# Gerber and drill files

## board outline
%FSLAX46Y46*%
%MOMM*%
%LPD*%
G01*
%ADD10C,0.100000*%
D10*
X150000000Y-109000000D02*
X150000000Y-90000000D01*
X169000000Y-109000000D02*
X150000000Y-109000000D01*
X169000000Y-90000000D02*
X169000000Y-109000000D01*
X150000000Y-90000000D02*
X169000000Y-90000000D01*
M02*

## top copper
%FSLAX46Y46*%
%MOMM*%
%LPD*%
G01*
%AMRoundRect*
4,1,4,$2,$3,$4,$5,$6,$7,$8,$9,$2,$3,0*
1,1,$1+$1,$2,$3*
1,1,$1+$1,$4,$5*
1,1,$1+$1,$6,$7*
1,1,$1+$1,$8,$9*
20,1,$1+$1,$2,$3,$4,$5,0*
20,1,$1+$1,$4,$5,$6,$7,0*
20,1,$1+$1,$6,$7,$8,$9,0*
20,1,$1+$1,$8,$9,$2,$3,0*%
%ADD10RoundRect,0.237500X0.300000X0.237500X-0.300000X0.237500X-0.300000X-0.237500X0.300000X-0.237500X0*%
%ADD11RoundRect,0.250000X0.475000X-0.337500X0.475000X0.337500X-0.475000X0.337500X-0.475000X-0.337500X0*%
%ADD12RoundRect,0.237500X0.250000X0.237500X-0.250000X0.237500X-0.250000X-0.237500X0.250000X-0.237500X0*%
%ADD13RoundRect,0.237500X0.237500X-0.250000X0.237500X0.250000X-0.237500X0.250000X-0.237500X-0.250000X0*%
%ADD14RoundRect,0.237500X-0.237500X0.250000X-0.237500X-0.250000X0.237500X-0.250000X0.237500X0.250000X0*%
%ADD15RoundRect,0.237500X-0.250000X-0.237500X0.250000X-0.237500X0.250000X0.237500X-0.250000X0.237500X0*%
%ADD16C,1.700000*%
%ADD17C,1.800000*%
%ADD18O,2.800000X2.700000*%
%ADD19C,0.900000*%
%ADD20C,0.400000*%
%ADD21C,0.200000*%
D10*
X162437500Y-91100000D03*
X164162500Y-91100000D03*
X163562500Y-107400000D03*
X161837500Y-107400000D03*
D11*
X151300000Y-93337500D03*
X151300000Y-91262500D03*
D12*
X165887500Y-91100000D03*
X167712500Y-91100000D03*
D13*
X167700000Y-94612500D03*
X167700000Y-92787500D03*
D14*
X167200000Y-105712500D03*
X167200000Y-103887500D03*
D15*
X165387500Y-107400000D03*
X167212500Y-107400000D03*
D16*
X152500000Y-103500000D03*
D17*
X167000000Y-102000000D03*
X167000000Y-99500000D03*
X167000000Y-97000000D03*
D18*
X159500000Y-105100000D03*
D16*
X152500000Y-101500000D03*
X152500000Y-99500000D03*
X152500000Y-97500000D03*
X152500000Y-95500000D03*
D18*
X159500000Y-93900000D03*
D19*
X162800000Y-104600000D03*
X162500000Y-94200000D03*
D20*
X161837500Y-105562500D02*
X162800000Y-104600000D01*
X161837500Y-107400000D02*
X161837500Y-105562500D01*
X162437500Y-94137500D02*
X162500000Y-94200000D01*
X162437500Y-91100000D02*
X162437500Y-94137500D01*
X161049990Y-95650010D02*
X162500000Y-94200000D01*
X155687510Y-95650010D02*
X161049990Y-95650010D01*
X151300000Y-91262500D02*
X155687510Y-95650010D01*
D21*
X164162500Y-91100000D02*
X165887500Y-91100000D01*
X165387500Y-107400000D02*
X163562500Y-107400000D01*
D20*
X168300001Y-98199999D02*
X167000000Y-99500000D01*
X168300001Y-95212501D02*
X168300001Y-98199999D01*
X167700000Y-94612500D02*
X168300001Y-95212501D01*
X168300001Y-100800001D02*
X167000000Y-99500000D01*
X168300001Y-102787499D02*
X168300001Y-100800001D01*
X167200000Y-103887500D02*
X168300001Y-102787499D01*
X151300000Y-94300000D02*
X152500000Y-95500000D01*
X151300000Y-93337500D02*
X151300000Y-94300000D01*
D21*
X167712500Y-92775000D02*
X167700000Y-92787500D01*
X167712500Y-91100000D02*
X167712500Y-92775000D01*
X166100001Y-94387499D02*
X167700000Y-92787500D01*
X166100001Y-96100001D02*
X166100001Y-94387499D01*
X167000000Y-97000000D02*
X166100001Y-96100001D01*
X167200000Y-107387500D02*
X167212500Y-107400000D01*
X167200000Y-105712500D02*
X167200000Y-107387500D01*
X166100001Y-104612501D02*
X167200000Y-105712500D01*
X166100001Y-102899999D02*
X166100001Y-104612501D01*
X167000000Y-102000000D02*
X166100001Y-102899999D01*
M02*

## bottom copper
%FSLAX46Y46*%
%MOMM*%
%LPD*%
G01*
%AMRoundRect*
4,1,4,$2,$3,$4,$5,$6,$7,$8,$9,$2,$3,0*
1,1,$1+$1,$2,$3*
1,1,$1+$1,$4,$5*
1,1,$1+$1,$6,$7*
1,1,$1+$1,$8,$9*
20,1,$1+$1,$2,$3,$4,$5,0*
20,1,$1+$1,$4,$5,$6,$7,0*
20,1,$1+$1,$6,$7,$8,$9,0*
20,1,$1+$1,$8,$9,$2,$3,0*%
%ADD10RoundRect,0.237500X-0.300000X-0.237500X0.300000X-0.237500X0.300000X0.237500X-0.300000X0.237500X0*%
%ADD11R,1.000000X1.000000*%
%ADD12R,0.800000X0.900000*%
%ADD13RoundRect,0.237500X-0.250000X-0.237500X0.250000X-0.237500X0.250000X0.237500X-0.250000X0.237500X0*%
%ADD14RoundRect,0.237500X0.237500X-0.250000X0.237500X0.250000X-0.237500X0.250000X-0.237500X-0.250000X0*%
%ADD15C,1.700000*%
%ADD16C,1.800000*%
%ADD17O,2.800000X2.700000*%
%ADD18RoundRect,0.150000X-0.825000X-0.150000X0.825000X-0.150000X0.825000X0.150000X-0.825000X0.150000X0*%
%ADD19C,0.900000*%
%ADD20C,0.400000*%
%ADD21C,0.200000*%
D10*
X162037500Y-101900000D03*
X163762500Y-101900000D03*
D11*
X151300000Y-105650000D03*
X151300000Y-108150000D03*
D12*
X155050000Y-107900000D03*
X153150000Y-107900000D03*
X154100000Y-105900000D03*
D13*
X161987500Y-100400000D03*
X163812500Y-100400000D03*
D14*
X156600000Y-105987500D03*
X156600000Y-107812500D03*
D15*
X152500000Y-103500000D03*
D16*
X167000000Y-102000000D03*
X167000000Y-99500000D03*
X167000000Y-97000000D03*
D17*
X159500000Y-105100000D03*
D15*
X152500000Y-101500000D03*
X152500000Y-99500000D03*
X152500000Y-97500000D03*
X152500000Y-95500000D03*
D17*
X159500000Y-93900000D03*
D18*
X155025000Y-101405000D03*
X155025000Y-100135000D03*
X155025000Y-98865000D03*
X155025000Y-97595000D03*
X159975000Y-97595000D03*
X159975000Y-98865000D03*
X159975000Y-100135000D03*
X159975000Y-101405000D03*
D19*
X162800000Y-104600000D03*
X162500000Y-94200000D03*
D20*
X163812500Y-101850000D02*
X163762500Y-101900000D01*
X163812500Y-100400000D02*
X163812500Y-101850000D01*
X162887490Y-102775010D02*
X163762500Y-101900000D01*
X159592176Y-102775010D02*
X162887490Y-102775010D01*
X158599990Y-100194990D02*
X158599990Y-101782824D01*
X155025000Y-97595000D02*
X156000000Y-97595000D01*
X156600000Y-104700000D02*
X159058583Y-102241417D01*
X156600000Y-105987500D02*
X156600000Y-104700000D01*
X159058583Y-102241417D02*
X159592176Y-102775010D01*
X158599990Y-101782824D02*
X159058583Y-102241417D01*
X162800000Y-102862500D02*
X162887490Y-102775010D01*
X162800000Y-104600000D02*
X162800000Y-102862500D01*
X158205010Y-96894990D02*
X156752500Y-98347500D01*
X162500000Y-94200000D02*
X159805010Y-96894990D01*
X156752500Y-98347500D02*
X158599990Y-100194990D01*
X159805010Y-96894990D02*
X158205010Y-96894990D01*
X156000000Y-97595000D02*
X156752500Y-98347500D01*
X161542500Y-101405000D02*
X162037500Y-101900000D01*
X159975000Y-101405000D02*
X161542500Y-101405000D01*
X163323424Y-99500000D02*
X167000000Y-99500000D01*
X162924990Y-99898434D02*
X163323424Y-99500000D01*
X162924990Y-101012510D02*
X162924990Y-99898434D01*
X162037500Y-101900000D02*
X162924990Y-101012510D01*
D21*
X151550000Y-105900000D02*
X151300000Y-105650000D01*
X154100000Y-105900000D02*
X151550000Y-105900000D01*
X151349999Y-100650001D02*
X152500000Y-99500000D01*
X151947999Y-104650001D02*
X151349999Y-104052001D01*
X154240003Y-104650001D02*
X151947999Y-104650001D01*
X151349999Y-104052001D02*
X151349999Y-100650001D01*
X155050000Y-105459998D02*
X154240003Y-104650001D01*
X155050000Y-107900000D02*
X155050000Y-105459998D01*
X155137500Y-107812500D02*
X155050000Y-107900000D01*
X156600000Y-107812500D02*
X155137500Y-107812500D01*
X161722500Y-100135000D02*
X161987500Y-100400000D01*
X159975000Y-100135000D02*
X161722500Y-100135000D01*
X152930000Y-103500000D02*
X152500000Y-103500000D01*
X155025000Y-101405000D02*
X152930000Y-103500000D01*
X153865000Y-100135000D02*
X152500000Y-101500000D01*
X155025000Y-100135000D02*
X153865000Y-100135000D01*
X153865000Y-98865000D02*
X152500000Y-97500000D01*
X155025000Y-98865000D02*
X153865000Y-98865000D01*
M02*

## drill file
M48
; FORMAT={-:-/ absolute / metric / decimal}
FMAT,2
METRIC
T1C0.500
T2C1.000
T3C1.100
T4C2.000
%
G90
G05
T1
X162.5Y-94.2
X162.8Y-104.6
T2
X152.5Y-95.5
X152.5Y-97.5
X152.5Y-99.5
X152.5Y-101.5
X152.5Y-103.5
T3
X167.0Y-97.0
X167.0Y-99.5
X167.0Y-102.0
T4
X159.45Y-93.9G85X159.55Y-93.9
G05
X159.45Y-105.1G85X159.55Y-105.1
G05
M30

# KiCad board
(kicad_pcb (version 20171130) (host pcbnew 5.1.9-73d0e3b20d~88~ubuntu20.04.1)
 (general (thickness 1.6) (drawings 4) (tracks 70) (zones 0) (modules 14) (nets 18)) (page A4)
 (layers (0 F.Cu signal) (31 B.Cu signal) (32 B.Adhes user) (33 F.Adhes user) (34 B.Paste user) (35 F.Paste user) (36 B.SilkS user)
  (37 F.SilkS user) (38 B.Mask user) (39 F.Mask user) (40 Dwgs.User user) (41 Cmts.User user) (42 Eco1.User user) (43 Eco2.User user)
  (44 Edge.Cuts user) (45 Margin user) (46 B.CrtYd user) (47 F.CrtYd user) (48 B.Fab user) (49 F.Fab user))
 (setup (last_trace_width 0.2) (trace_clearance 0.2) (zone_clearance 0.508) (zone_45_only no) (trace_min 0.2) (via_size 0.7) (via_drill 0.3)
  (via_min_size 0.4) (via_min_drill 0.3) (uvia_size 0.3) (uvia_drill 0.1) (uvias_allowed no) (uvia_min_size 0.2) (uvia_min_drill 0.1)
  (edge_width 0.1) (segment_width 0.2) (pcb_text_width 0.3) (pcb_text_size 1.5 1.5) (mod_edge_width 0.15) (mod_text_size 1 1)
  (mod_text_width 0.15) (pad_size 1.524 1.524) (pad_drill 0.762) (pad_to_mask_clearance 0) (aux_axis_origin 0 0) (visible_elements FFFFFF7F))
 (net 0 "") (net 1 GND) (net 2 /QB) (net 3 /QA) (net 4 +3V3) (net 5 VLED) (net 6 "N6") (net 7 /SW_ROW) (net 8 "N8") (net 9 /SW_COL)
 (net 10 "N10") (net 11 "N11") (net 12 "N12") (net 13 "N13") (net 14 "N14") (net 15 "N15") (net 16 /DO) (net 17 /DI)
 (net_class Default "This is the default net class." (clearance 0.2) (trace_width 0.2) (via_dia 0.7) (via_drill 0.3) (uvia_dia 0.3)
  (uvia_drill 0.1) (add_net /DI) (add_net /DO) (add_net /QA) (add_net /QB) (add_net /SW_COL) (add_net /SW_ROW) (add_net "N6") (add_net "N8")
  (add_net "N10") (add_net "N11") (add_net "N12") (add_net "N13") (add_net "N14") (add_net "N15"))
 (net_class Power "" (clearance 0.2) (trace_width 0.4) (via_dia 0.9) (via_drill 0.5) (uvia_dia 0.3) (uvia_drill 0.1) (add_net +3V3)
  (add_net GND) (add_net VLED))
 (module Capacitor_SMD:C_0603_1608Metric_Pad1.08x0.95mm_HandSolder (layer F.Cu) (at 163.3 91.1 180)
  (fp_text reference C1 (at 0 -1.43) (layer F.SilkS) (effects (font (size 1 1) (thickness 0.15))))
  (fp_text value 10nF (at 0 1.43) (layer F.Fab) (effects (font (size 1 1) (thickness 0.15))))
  (pad 2 smd roundrect (at 0.8625 0 180) (size 1.075 0.95) (layers F.Cu F.Paste F.Mask) (roundrect_rratio 0.25) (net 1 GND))
  (pad 1 smd roundrect (at -0.8625 0 180) (size 1.075 0.95) (layers F.Cu F.Paste F.Mask) (roundrect_rratio 0.25) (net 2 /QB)))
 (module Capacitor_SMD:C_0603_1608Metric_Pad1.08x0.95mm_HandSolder (layer F.Cu) (at 162.7 107.4 180)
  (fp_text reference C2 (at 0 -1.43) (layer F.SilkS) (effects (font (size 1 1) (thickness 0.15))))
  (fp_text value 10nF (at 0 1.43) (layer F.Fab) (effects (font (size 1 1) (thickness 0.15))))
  (pad 1 smd roundrect (at -0.8625 0 180) (size 1.075 0.95) (layers F.Cu F.Paste F.Mask) (roundrect_rratio 0.25) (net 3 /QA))
  (pad 2 smd roundrect (at 0.8625 0 180) (size 1.075 0.95) (layers F.Cu F.Paste F.Mask) (roundrect_rratio 0.25) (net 1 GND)))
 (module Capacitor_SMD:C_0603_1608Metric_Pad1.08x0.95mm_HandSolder (layer B.Cu) (at 162.9 101.9)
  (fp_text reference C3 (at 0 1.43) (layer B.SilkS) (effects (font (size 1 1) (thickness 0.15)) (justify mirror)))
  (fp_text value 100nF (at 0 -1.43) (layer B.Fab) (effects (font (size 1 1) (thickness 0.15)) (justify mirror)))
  (pad 1 smd roundrect (at -0.8625 0) (size 1.075 0.95) (layers B.Cu B.Paste B.Mask) (roundrect_rratio 0.25) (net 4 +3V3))
  (pad 2 smd roundrect (at 0.8625 0) (size 1.075 0.95) (layers B.Cu B.Paste B.Mask) (roundrect_rratio 0.25) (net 1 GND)))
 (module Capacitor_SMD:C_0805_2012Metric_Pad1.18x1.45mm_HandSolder (layer F.Cu) (at 151.3 92.3 90)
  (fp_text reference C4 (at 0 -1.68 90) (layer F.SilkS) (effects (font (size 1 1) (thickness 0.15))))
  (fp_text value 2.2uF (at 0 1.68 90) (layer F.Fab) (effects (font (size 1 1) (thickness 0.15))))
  (pad 1 smd roundrect (at -1.0375 0 90) (size 1.175 1.45) (layers F.Cu F.Paste F.Mask) (roundrect_rratio 0.212766) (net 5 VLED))
  (pad 2 smd roundrect (at 1.0375 0 90) (size 1.175 1.45) (layers F.Cu F.Paste F.Mask) (roundrect_rratio 0.212766) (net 1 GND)))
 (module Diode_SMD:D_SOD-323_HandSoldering (layer B.Cu) (at 151.3 106.9 270)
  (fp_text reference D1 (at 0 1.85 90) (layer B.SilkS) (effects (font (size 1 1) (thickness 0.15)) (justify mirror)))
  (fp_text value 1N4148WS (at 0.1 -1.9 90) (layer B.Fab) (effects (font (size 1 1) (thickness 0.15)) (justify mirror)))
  (pad 1 smd rect (at -1.25 0 270) (size 1 1) (layers B.Cu B.Paste B.Mask) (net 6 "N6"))
  (pad 2 smd rect (at 1.25 0 270) (size 1 1) (layers B.Cu B.Paste B.Mask) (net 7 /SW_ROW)))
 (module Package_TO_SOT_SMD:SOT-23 (layer B.Cu) (at 154.1 106.9 90)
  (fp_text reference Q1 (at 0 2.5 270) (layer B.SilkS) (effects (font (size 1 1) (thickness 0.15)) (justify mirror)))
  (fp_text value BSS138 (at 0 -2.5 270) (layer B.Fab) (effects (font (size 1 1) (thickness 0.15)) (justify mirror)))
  (pad 1 smd rect (at -1 0.95 90) (size 0.9 0.8) (layers B.Cu B.Paste B.Mask) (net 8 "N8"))
  (pad 2 smd rect (at -1 -0.95 90) (size 0.9 0.8) (layers B.Cu B.Paste B.Mask) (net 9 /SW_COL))
  (pad 3 smd rect (at 1 0 90) (size 0.9 0.8) (layers B.Cu B.Paste B.Mask) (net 6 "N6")))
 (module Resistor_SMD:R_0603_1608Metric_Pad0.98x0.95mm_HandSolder (layer F.Cu) (at 166.8 91.1 180)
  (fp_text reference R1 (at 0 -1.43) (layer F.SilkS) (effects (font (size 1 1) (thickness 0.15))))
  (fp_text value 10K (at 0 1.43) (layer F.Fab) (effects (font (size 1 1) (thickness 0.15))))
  (pad 2 smd roundrect (at 0.9125 0 180) (size 0.975 0.95) (layers F.Cu F.Paste F.Mask) (roundrect_rratio 0.25) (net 2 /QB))
  (pad 1 smd roundrect (at -0.9125 0 180) (size 0.975 0.95) (layers F.Cu F.Paste F.Mask) (roundrect_rratio 0.25) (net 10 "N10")))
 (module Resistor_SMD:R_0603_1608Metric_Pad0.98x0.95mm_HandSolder (layer F.Cu) (at 167.7 93.7 90)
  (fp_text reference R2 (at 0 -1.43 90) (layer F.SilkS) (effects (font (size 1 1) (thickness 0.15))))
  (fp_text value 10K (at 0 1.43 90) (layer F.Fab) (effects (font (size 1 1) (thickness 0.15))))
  (pad 1 smd roundrect (at -0.9125 0 90) (size 0.975 0.95) (layers F.Cu F.Paste F.Mask) (roundrect_rratio 0.25) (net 4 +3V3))
  (pad 2 smd roundrect (at 0.9125 0 90) (size 0.975 0.95) (layers F.Cu F.Paste F.Mask) (roundrect_rratio 0.25) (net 10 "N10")))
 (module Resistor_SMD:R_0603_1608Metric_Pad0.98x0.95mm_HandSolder (layer B.Cu) (at 162.9 100.4)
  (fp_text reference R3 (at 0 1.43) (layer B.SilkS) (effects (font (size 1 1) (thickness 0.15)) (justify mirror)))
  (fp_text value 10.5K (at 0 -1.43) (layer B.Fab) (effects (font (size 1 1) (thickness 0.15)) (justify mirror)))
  (pad 1 smd roundrect (at -0.9125 0) (size 0.975 0.95) (layers B.Cu B.Paste B.Mask) (roundrect_rratio 0.25) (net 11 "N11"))
  (pad 2 smd roundrect (at 0.9125 0) (size 0.975 0.95) (layers B.Cu B.Paste B.Mask) (roundrect_rratio 0.25) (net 1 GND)))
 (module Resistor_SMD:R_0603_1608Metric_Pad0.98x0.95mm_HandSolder (layer F.Cu) (at 167.2 104.8 270)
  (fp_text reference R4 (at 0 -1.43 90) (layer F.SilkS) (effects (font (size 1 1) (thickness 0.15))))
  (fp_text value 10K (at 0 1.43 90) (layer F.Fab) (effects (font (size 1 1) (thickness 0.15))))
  (pad 2 smd roundrect (at 0.9125 0 270) (size 0.975 0.95) (layers F.Cu F.Paste F.Mask) (roundrect_rratio 0.25) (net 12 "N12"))
  (pad 1 smd roundrect (at -0.9125 0 270) (size 0.975 0.95) (layers F.Cu F.Paste F.Mask) (roundrect_rratio 0.25) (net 4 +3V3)))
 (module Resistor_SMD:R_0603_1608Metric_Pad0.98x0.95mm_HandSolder (layer F.Cu) (at 166.3 107.4)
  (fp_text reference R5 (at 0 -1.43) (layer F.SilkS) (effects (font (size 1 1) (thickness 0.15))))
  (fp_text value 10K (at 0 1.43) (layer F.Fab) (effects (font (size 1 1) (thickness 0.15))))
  (pad 1 smd roundrect (at -0.9125 0) (size 0.975 0.95) (layers F.Cu F.Paste F.Mask) (roundrect_rratio 0.25) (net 3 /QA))
  (pad 2 smd roundrect (at 0.9125 0) (size 0.975 0.95) (layers F.Cu F.Paste F.Mask) (roundrect_rratio 0.25) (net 12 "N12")))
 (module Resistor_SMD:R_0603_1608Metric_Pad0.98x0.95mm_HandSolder (layer B.Cu) (at 156.6 106.9 90)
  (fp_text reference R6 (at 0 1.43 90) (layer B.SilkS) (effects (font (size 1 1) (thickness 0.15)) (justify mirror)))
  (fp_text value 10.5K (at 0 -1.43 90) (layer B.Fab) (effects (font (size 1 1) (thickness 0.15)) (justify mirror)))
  (pad 2 smd roundrect (at 0.9125 0 90) (size 0.975 0.95) (layers B.Cu B.Paste B.Mask) (roundrect_rratio 0.25) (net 1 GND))
  (pad 1 smd roundrect (at -0.9125 0 90) (size 0.975 0.95) (layers B.Cu B.Paste B.Mask) (roundrect_rratio 0.25) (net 8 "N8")))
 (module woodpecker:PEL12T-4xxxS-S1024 (layer F.Cu) (at 159.5 99.5 90)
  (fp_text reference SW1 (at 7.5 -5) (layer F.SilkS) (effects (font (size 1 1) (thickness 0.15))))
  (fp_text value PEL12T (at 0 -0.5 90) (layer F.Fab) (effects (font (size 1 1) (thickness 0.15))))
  (pad 1 thru_hole circle (at -4 -7 90) (size 1.7 1.7) (drill 1) (layers *.Cu *.Mask) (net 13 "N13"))
  (pad A thru_hole circle (at -2.5 7.5 90) (size 1.8 1.8) (drill 1.1) (layers *.Cu *.Mask) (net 12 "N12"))
  (pad C thru_hole circle (at 0 7.5 90) (size 1.8 1.8) (drill 1.1) (layers *.Cu *.Mask) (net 4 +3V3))
  (pad B thru_hole circle (at 2.5 7.5 90) (size 1.8 1.8) (drill 1.1) (layers *.Cu *.Mask) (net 10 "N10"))
  (pad "" np_thru_hole oval (at -5.6 0 90) (size 2.7 2.8) (drill oval 2 2.1) (layers *.Cu *.Mask))
  (pad 2 thru_hole circle (at -2 -7 90) (size 1.7 1.7) (drill 1) (layers *.Cu *.Mask) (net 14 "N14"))
  (pad 3 thru_hole circle (at 0 -7 90) (size 1.7 1.7) (drill 1) (layers *.Cu *.Mask) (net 8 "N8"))
  (pad 4 thru_hole circle (at 2 -7 90) (size 1.7 1.7) (drill 1) (layers *.Cu *.Mask) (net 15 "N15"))
  (pad 5 thru_hole circle (at 4 -7 90) (size 1.7 1.7) (drill 1) (layers *.Cu *.Mask) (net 5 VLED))
  (pad "" np_thru_hole oval (at 5.6 0 90) (size 2.7 2.8) (drill oval 2 2.1) (layers *.Cu *.Mask)))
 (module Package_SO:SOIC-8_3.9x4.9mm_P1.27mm (layer B.Cu) (at 157.5 99.5)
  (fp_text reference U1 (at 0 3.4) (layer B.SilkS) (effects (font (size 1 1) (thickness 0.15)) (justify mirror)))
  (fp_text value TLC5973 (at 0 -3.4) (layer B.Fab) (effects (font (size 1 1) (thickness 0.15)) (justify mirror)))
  (pad 1 smd roundrect (at -2.475 1.905) (size 1.95 0.6) (layers B.Cu B.Paste B.Mask) (roundrect_rratio 0.25) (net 13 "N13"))
  (pad 2 smd roundrect (at -2.475 0.635) (size 1.95 0.6) (layers B.Cu B.Paste B.Mask) (roundrect_rratio 0.25) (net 14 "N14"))
  (pad 3 smd roundrect (at -2.475 -0.635) (size 1.95 0.6) (layers B.Cu B.Paste B.Mask) (roundrect_rratio 0.25) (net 15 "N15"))
  (pad 4 smd roundrect (at -2.475 -1.905) (size 1.95 0.6) (layers B.Cu B.Paste B.Mask) (roundrect_rratio 0.25) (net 1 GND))
  (pad 5 smd roundrect (at 2.475 -1.905) (size 1.95 0.6) (layers B.Cu B.Paste B.Mask) (roundrect_rratio 0.25) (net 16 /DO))
  (pad 6 smd roundrect (at 2.475 -0.635) (size 1.95 0.6) (layers B.Cu B.Paste B.Mask) (roundrect_rratio 0.25) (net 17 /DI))
  (pad 7 smd roundrect (at 2.475 0.635) (size 1.95 0.6) (layers B.Cu B.Paste B.Mask) (roundrect_rratio 0.25) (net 11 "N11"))
  (pad 8 smd roundrect (at 2.475 1.905) (size 1.95 0.6) (layers B.Cu B.Paste B.Mask) (roundrect_rratio 0.25) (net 4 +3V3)))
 (gr_line (start 150 109) (end 150 90) (layer Edge.Cuts) (width 0.1))
 (gr_line (start 169 109) (end 150 109) (layer Edge.Cuts) (width 0.1))
 (gr_line (start 169 90) (end 169 109) (layer Edge.Cuts) (width 0.1))
 (gr_line (start 150 90) (end 169 90) (layer Edge.Cuts) (width 0.1))
 (segment (start 163.8125 101.85) (end 163.7625 101.9) (width 0.4) (layer B.Cu) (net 1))
 (segment (start 163.8125 100.4) (end 163.8125 101.85) (width 0.4) (layer B.Cu) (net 1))
 (segment (start 162.88749 102.77501) (end 163.7625 101.9) (width 0.4) (layer B.Cu) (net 1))
 (segment (start 159.592176 102.77501) (end 162.88749 102.77501) (width 0.4) (layer B.Cu) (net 1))
 (segment (start 158.59999 100.19499) (end 158.59999 101.782824) (width 0.4) (layer B.Cu) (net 1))
 (segment (start 155.025 97.595) (end 156 97.595) (width 0.4) (layer B.Cu) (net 1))
 (segment (start 156.6 104.7) (end 159.058583 102.241417) (width 0.4) (layer B.Cu) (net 1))
 (segment (start 156.6 105.9875) (end 156.6 104.7) (width 0.4) (layer B.Cu) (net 1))
 (segment (start 159.058583 102.241417) (end 159.592176 102.77501) (width 0.4) (layer B.Cu) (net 1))
 (segment (start 158.59999 101.782824) (end 159.058583 102.241417) (width 0.4) (layer B.Cu) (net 1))
 (via (at 162.8 104.6) (size 0.9) (drill 0.5) (layers F.Cu B.Cu) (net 1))
 (segment (start 161.8375 105.5625) (end 162.8 104.6) (width 0.4) (layer F.Cu) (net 1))
 (segment (start 161.8375 107.4) (end 161.8375 105.5625) (width 0.4) (layer F.Cu) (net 1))
 (segment (start 162.8 102.8625) (end 162.88749 102.77501) (width 0.4) (layer B.Cu) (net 1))
 (segment (start 162.8 104.6) (end 162.8 102.8625) (width 0.4) (layer B.Cu) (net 1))
 (via (at 162.5 94.2) (size 0.9) (drill 0.5) (layers F.Cu B.Cu) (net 1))
 (segment (start 162.4375 94.1375) (end 162.5 94.2) (width 0.4) (layer F.Cu) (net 1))
 (segment (start 162.4375 91.1) (end 162.4375 94.1375) (width 0.4) (layer F.Cu) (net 1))
 (segment (start 158.20501 96.89499) (end 156.7525 98.3475) (width 0.4) (layer B.Cu) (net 1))
 (segment (start 162.5 94.2) (end 159.80501 96.89499) (width 0.4) (layer B.Cu) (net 1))
 (segment (start 156.7525 98.3475) (end 158.59999 100.19499) (width 0.4) (layer B.Cu) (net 1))
 (segment (start 159.80501 96.89499) (end 158.20501 96.89499) (width 0.4) (layer B.Cu) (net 1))
 (segment (start 156 97.595) (end 156.7525 98.3475) (width 0.4) (layer B.Cu) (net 1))
 (segment (start 161.04999 95.65001) (end 162.5 94.2) (width 0.4) (layer F.Cu) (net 1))
 (segment (start 155.68751 95.65001) (end 161.04999 95.65001) (width 0.4) (layer F.Cu) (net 1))
 (segment (start 151.3 91.2625) (end 155.68751 95.65001) (width 0.4) (layer F.Cu) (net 1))
 (segment (start 164.1625 91.1) (end 165.8875 91.1) (width 0.2) (layer F.Cu) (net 2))
 (segment (start 165.3875 107.4) (end 163.5625 107.4) (width 0.2) (layer F.Cu) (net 3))
 (segment (start 161.5425 101.405) (end 162.0375 101.9) (width 0.4) (layer B.Cu) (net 4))
 (segment (start 159.975 101.405) (end 161.5425 101.405) (width 0.4) (layer B.Cu) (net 4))
 (segment (start 163.323424 99.5) (end 167 99.5) (width 0.4) (layer B.Cu) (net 4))
 (segment (start 162.92499 99.898434) (end 163.323424 99.5) (width 0.4) (layer B.Cu) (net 4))
 (segment (start 162.92499 101.01251) (end 162.92499 99.898434) (width 0.4) (layer B.Cu) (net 4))
 (segment (start 162.0375 101.9) (end 162.92499 101.01251) (width 0.4) (layer B.Cu) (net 4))
 (segment (start 168.300001 98.199999) (end 167 99.5) (width 0.4) (layer F.Cu) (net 4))
 (segment (start 168.300001 95.212501) (end 168.300001 98.199999) (width 0.4) (layer F.Cu) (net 4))
 (segment (start 167.7 94.6125) (end 168.300001 95.212501) (width 0.4) (layer F.Cu) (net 4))
 (segment (start 168.300001 100.800001) (end 167 99.5) (width 0.4) (layer F.Cu) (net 4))
 (segment (start 168.300001 102.787499) (end 168.300001 100.800001) (width 0.4) (layer F.Cu) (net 4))
 (segment (start 167.2 103.8875) (end 168.300001 102.787499) (width 0.4) (layer F.Cu) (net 4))
 (segment (start 151.3 94.3) (end 152.5 95.5) (width 0.4) (layer F.Cu) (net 5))
 (segment (start 151.3 93.3375) (end 151.3 94.3) (width 0.4) (layer F.Cu) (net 5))
 (segment (start 151.55 105.9) (end 151.3 105.65) (width 0.2) (layer B.Cu) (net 6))
 (segment (start 154.1 105.9) (end 151.55 105.9) (width 0.2) (layer B.Cu) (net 6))
 (segment (start 151.349999 100.650001) (end 152.5 99.5) (width 0.2) (layer B.Cu) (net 8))
 (segment (start 151.947999 104.650001) (end 151.349999 104.052001) (width 0.2) (layer B.Cu) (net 8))
 (segment (start 154.240003 104.650001) (end 151.947999 104.650001) (width 0.2) (layer B.Cu) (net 8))
 (segment (start 151.349999 104.052001) (end 151.349999 100.650001) (width 0.2) (layer B.Cu) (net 8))
 (segment (start 155.05 105.459998) (end 154.240003 104.650001) (width 0.2) (layer B.Cu) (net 8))
 (segment (start 155.05 107.9) (end 155.05 105.459998) (width 0.2) (layer B.Cu) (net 8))
 (segment (start 155.1375 107.8125) (end 155.05 107.9) (width 0.2) (layer B.Cu) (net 8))
 (segment (start 156.6 107.8125) (end 155.1375 107.8125) (width 0.2) (layer B.Cu) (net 8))
 (segment (start 167.7125 92.775) (end 167.7 92.7875) (width 0.2) (layer F.Cu) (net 10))
 (segment (start 167.7125 91.1) (end 167.7125 92.775) (width 0.2) (layer F.Cu) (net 10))
 (segment (start 166.100001 94.387499) (end 167.7 92.7875) (width 0.2) (layer F.Cu) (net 10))
 (segment (start 166.100001 96.100001) (end 166.100001 94.387499) (width 0.2) (layer F.Cu) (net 10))
 (segment (start 167 97) (end 166.100001 96.100001) (width 0.2) (layer F.Cu) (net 10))
 (segment (start 161.7225 100.135) (end 161.9875 100.4) (width 0.2) (layer B.Cu) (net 11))
 (segment (start 159.975 100.135) (end 161.7225 100.135) (width 0.2) (layer B.Cu) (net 11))
 (segment (start 167.2 107.3875) (end 167.2125 107.4) (width 0.2) (layer F.Cu) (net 12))
 (segment (start 167.2 105.7125) (end 167.2 107.3875) (width 0.2) (layer F.Cu) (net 12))
 (segment (start 166.100001 104.612501) (end 167.2 105.7125) (width 0.2) (layer F.Cu) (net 12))
 (segment (start 166.100001 102.899999) (end 166.100001 104.612501) (width 0.2) (layer F.Cu) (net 12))
 (segment (start 167 102) (end 166.100001 102.899999) (width 0.2) (layer F.Cu) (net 12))
 (segment (start 152.93 103.5) (end 152.5 103.5) (width 0.2) (layer B.Cu) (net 13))
 (segment (start 155.025 101.405) (end 152.93 103.5) (width 0.2) (layer B.Cu) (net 13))
 (segment (start 153.865 100.135) (end 152.5 101.5) (width 0.2) (layer B.Cu) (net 14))
 (segment (start 155.025 100.135) (end 153.865 100.135) (width 0.2) (layer B.Cu) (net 14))
 (segment (start 153.865 98.865) (end 152.5 97.5) (width 0.2) (layer B.Cu) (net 15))
 (segment (start 155.025 98.865) (end 153.865 98.865) (width 0.2) (layer B.Cu) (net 15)))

